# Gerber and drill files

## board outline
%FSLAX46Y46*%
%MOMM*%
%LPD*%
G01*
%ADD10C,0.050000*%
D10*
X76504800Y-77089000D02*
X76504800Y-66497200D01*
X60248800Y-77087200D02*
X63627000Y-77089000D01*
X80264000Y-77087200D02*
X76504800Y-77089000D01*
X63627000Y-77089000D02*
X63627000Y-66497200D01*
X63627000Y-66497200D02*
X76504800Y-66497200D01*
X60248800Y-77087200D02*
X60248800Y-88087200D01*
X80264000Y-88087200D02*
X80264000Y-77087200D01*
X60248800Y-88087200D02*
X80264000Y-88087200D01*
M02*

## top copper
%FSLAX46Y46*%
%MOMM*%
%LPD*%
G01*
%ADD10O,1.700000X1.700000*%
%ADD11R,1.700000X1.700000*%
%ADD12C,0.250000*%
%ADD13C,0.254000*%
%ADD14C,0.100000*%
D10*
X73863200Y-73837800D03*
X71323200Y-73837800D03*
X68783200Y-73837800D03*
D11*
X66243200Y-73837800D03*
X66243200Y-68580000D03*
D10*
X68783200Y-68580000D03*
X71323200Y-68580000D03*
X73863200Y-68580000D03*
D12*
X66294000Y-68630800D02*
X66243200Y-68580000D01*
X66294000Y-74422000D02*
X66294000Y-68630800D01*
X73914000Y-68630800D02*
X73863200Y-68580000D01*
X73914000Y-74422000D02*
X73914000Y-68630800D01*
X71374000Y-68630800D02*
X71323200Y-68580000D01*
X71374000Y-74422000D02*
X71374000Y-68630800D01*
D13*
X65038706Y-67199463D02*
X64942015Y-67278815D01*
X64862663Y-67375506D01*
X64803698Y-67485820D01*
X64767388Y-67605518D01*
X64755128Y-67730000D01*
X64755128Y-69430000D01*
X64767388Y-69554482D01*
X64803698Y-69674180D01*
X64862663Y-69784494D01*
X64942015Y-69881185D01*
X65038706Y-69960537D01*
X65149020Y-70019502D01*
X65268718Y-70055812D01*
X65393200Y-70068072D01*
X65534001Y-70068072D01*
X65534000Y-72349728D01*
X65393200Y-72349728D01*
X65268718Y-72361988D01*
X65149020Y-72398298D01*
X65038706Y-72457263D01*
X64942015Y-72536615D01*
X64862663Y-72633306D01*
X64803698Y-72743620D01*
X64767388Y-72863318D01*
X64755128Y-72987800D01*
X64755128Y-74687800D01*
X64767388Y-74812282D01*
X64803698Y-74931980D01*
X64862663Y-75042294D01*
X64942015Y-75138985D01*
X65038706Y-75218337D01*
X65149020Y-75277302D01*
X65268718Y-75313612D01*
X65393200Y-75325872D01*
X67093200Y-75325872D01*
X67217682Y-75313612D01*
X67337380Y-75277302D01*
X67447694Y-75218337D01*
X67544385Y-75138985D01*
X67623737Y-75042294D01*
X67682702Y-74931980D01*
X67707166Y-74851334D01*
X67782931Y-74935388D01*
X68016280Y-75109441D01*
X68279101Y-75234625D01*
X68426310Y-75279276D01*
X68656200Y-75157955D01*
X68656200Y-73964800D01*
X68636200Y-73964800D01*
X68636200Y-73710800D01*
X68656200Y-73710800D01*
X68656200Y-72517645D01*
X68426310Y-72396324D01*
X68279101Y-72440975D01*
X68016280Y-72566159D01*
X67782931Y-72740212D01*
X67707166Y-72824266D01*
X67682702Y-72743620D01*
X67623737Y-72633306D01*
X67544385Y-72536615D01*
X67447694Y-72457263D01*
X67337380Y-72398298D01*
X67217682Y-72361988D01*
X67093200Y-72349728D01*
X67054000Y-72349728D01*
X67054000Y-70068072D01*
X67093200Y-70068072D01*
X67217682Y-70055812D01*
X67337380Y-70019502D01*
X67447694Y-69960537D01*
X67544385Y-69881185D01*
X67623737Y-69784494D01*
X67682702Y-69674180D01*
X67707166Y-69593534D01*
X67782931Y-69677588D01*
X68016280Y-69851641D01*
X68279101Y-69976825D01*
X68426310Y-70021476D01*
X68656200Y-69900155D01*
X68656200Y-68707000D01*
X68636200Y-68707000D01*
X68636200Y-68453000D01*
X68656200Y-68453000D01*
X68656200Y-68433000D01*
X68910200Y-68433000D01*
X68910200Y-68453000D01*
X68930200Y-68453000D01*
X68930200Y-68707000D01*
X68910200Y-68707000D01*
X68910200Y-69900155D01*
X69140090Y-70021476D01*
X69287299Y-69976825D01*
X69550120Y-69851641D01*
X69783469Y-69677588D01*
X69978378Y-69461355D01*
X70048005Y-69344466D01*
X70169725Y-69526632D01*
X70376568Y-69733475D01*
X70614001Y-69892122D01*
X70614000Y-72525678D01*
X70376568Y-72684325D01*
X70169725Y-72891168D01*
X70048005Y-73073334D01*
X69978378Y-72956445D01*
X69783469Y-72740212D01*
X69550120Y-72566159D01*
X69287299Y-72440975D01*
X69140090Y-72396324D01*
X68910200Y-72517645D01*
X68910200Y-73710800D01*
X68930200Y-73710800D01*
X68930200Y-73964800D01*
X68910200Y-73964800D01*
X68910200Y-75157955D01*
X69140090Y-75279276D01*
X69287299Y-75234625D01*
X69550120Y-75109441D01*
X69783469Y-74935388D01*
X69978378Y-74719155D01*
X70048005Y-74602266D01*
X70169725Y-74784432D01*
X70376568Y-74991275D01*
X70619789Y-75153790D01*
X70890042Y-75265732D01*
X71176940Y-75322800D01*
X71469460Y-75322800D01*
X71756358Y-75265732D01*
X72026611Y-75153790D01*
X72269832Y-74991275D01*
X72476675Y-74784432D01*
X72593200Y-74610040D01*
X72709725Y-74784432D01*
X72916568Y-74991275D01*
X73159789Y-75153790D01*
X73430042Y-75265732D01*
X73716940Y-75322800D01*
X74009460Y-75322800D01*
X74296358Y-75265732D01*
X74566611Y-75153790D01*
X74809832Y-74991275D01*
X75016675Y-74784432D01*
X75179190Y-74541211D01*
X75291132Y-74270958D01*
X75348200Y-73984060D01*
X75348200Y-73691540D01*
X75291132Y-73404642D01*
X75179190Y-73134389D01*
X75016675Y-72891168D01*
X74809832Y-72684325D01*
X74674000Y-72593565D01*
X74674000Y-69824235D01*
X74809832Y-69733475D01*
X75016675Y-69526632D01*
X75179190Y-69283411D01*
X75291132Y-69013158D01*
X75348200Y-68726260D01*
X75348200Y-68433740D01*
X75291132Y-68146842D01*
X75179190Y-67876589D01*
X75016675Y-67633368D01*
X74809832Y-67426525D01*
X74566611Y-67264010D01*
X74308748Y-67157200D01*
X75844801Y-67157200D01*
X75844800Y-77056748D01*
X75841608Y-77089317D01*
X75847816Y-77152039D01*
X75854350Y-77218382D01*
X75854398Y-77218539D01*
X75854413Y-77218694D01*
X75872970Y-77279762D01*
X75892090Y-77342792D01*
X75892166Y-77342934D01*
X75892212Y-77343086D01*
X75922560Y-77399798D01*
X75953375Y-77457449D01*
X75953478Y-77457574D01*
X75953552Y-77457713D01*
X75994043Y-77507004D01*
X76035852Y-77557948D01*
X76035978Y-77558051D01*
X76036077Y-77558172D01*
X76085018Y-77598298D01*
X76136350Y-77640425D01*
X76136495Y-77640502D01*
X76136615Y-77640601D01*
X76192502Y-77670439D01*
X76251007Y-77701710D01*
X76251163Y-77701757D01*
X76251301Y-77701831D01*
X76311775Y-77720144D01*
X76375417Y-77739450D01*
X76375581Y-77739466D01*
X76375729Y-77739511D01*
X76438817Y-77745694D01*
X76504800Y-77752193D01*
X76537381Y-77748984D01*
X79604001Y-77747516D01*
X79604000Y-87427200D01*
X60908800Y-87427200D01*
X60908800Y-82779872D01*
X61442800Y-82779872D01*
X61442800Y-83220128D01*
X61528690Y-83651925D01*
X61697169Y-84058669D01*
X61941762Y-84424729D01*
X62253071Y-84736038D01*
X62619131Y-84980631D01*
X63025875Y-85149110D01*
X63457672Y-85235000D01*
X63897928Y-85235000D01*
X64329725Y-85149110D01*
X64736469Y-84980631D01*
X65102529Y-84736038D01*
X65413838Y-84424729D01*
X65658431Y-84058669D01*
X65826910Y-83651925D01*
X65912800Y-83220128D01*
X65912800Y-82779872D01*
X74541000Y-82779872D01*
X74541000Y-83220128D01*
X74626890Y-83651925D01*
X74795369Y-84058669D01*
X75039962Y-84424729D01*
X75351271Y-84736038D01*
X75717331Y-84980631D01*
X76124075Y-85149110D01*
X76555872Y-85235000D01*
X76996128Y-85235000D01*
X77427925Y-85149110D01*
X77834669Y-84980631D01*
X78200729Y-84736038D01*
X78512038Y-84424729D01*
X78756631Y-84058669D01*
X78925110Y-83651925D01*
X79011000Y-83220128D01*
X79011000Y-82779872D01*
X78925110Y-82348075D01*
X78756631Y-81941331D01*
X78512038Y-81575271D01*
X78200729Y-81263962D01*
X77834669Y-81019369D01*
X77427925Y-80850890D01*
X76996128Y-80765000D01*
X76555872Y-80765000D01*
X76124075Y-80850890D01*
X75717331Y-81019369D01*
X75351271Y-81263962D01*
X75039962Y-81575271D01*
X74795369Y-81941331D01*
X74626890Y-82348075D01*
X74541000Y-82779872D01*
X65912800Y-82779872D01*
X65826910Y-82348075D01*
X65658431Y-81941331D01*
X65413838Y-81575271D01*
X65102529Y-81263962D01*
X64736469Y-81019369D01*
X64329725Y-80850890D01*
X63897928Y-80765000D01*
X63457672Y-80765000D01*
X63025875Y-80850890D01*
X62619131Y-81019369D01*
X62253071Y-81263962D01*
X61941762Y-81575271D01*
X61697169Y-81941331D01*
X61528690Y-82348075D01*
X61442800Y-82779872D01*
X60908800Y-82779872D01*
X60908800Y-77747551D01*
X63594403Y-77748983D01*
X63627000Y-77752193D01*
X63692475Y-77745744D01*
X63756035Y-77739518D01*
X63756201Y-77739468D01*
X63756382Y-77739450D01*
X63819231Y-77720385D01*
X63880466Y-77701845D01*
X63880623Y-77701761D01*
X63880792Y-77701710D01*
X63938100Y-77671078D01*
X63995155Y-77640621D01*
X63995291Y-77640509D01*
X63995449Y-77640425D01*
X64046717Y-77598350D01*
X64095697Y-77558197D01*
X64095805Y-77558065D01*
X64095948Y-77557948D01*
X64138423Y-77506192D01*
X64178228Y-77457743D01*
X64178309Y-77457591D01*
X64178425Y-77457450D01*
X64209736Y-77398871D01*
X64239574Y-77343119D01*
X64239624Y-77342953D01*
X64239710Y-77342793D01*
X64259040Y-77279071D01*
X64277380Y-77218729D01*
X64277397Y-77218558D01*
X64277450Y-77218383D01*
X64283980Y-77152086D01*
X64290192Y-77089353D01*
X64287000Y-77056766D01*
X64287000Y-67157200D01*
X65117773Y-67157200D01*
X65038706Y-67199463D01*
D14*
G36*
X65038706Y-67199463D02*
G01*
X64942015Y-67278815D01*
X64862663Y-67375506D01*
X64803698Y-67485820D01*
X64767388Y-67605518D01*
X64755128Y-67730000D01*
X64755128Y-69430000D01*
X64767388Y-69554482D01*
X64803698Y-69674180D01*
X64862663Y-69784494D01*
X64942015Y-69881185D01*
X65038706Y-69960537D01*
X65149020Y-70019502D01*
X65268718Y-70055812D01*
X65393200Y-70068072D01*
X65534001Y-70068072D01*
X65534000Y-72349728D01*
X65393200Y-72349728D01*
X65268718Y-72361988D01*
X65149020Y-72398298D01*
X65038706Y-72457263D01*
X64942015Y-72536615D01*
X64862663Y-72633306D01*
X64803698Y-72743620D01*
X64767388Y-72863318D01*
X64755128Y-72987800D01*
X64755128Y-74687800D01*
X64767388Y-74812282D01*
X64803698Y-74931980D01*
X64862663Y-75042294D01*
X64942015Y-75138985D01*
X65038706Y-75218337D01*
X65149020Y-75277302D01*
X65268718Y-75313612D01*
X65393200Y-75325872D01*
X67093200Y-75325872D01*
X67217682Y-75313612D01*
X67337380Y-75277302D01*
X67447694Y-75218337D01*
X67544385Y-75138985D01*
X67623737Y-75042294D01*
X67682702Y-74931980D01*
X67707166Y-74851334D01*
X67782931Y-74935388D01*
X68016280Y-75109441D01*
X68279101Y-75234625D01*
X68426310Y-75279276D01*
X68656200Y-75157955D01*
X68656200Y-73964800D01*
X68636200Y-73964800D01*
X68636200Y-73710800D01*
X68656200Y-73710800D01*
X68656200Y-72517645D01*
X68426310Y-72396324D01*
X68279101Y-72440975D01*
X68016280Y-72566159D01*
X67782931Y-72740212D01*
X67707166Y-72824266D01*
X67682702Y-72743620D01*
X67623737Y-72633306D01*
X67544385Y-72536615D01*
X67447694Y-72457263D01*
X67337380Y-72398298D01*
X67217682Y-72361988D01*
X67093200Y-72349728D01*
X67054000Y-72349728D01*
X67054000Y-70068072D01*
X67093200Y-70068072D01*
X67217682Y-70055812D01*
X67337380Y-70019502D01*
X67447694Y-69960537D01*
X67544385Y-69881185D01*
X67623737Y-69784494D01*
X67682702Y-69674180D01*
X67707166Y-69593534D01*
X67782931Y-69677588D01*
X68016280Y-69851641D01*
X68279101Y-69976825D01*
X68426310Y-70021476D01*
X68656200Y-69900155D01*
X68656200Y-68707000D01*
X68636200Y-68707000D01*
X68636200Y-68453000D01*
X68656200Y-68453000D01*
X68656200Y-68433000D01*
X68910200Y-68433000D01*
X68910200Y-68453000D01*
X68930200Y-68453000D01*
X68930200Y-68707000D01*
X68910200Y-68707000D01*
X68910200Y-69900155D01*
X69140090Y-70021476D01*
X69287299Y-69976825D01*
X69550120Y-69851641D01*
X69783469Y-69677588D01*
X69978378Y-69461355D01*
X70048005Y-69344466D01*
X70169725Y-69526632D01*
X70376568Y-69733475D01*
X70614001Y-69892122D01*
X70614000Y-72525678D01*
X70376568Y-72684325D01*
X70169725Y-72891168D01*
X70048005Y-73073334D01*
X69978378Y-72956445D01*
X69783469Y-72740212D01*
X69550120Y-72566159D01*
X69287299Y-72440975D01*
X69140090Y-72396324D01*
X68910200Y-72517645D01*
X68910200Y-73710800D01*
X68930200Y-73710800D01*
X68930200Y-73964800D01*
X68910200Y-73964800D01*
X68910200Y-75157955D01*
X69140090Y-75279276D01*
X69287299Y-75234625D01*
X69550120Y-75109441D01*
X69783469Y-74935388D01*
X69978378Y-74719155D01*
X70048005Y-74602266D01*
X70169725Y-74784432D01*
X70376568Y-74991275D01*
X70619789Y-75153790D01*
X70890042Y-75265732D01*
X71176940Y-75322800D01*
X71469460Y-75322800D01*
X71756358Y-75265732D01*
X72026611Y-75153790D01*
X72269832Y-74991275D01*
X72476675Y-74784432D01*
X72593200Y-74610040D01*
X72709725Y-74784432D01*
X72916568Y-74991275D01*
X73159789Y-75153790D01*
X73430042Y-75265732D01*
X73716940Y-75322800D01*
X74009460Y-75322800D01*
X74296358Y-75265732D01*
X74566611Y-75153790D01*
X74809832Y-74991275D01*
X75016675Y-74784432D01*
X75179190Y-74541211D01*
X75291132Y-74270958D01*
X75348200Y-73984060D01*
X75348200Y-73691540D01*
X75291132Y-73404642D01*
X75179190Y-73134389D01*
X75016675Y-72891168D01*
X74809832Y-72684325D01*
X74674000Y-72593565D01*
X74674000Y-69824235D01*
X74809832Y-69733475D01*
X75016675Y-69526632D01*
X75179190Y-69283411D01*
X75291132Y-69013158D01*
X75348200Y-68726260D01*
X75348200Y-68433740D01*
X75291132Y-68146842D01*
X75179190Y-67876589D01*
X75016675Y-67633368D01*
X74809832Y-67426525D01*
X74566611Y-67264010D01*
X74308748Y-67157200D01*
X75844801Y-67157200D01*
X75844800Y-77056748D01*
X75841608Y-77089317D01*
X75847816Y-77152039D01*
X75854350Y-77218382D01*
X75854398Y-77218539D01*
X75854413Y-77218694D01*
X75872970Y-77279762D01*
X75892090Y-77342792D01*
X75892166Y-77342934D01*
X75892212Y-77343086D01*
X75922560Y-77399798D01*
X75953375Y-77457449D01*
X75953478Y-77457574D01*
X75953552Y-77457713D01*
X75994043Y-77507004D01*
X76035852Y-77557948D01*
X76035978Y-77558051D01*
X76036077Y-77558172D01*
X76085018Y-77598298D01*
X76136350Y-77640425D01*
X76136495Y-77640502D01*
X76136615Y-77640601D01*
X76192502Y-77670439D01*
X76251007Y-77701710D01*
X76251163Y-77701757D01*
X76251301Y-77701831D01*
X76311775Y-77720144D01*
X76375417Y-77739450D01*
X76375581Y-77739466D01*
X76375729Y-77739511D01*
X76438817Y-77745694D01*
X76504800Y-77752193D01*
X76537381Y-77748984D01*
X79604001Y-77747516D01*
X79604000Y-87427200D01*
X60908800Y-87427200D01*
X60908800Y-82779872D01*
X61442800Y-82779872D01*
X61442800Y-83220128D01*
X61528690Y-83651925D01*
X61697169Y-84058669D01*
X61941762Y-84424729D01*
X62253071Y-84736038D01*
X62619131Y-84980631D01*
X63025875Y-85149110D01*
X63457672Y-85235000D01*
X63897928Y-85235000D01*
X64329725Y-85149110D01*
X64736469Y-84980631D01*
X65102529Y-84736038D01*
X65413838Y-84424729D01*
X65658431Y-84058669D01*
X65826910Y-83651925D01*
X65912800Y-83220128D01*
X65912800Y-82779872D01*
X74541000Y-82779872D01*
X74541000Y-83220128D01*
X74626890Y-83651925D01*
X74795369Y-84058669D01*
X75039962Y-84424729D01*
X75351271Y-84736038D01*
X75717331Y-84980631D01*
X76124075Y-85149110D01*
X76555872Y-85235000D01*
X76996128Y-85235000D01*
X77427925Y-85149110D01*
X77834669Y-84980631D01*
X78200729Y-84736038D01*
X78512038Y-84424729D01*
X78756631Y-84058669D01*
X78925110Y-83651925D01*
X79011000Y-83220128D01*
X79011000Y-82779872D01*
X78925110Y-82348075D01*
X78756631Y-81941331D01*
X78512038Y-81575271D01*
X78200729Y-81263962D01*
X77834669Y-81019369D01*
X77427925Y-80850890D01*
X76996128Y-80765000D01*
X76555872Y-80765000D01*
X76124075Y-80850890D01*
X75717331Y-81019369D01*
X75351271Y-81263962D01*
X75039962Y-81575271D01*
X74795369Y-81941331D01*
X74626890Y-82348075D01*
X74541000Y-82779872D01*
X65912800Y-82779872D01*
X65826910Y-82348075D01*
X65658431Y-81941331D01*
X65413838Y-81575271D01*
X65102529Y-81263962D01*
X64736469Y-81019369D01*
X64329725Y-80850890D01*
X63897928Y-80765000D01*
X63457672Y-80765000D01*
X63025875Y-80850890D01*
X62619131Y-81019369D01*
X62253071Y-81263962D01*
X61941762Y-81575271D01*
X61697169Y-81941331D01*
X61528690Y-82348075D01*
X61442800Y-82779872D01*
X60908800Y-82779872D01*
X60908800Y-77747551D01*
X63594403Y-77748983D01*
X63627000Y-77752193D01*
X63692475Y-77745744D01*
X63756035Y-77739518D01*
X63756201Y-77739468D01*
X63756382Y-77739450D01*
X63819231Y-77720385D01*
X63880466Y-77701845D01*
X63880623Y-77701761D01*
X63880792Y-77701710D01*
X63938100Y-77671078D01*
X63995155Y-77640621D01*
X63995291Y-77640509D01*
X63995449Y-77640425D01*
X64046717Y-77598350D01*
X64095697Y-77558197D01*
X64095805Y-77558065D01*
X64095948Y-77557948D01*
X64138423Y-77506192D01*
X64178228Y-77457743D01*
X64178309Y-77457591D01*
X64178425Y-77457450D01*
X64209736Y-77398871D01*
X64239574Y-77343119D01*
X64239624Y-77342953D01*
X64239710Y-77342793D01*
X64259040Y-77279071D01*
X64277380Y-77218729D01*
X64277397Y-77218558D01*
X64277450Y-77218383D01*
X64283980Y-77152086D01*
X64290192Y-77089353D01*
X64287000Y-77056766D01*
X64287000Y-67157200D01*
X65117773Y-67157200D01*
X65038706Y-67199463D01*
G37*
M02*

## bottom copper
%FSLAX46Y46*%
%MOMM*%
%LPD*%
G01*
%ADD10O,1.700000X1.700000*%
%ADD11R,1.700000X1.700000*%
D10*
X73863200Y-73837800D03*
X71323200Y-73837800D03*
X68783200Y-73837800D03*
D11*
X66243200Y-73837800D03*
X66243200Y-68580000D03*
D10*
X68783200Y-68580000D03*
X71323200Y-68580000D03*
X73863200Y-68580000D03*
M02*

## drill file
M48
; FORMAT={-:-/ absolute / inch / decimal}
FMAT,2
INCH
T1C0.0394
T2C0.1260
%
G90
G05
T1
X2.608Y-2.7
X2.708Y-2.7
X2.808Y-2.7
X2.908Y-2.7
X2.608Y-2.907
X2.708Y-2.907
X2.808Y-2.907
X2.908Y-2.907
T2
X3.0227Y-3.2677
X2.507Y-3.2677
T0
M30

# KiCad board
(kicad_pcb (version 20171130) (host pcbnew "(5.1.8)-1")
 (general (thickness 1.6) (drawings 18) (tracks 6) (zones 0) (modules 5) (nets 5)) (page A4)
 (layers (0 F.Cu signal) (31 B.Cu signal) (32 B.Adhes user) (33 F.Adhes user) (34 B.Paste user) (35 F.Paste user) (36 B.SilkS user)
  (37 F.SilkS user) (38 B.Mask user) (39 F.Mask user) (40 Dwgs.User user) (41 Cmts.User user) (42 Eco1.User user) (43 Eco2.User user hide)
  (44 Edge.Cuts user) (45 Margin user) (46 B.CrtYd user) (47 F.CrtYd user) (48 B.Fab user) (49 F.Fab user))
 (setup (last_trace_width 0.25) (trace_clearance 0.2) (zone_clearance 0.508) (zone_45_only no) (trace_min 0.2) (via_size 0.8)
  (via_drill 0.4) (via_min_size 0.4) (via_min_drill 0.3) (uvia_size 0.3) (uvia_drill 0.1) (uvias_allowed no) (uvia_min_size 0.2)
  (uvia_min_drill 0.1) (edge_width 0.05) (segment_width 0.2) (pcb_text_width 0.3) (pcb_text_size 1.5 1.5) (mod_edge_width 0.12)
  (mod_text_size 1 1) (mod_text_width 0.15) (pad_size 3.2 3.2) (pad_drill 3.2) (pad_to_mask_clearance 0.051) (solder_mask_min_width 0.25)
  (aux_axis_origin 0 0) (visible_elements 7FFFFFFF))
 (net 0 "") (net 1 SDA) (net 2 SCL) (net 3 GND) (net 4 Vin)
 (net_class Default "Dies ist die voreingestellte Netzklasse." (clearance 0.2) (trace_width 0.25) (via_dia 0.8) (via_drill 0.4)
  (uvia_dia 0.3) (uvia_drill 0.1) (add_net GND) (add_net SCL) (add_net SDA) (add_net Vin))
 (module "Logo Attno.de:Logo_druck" (layer F.Cu) (at 70.0786 81.6356)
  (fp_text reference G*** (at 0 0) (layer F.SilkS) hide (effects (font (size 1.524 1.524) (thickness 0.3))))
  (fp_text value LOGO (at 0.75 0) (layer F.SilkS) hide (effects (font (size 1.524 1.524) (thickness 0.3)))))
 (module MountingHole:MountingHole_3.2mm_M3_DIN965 (layer F.Cu) (at 76.776 83)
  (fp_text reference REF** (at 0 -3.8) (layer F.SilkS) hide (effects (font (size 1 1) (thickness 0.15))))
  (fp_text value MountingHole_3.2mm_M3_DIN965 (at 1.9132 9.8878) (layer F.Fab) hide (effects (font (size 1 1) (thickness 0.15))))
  (pad 1 np_thru_hole circle (at 0 0) (size 3.2 3.2) (drill 3.2) (layers *.Cu *.Mask)))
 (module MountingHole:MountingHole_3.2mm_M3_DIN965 (layer F.Cu) (at 63.6778 83)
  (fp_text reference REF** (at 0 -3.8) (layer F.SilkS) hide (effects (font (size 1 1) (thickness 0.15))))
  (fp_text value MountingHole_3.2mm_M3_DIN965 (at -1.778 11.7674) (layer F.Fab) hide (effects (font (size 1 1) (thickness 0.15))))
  (pad 1 np_thru_hole circle (at 0 0) (size 3.2 3.2) (drill 3.2) (layers *.Cu *.Mask)))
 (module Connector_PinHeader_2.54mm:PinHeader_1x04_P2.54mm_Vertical (layer F.Cu) (at 66.2432 73.8378 90)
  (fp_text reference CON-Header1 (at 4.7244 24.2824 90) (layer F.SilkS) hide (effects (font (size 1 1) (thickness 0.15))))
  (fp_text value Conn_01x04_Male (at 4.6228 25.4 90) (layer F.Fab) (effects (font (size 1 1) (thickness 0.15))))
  (pad 4 thru_hole oval (at 0 7.62 90) (size 1.7 1.7) (drill 1) (layers *.Cu *.Mask) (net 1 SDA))
  (pad 3 thru_hole oval (at 0 5.08 90) (size 1.7 1.7) (drill 1) (layers *.Cu *.Mask) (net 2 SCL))
  (pad 2 thru_hole oval (at 0 2.54 90) (size 1.7 1.7) (drill 1) (layers *.Cu *.Mask) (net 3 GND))
  (pad 1 thru_hole rect (at 0 0 90) (size 1.7 1.7) (drill 1) (layers *.Cu *.Mask) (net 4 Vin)))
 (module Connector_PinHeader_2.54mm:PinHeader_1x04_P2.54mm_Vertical (layer F.Cu) (at 66.2432 68.58 90)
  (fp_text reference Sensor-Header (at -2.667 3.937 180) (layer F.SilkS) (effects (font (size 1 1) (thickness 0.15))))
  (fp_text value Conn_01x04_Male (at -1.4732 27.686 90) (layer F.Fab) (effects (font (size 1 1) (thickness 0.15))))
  (pad 1 thru_hole rect (at 0 0 90) (size 1.7 1.7) (drill 1) (layers *.Cu *.Mask) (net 4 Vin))
  (pad 2 thru_hole oval (at 0 2.54 90) (size 1.7 1.7) (drill 1) (layers *.Cu *.Mask) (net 3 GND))
  (pad 3 thru_hole oval (at 0 5.08 90) (size 1.7 1.7) (drill 1) (layers *.Cu *.Mask) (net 2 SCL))
  (pad 4 thru_hole oval (at 0 7.62 90) (size 1.7 1.7) (drill 1) (layers *.Cu *.Mask) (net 1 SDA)))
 (gr_line (start 76.5048 77.089) (end 76.5048 66.4972) (layer Edge.Cuts) (width 0.05))
 (gr_line (start 60.2488 77.0872) (end 63.627 77.089) (layer Edge.Cuts) (width 0.05))
 (gr_line (start 80.264 77.0872) (end 76.5048 77.089) (layer Edge.Cuts) (width 0.05))
 (gr_line (start 63.627 77.089) (end 63.627 66.4972) (layer Edge.Cuts) (width 0.05))
 (gr_line (start 63.627 66.4972) (end 76.5048 66.4972) (layer Edge.Cuts) (width 0.05))
 (gr_line (start 60.2488 77.0872) (end 60.2488 88.0872) (layer Edge.Cuts) (width 0.05))
 (gr_line (start 80.264 88.0872) (end 80.264 77.0872) (layer Edge.Cuts) (width 0.05))
 (gr_line (start 60.2488 88.0872) (end 80.264 88.0872) (layer Edge.Cuts) (width 0.05))
 (segment (start 66.294 68.6308) (end 66.2432 68.58) (width 0.25) (layer F.Cu) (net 4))
 (segment (start 66.294 74.422) (end 66.294 68.6308) (width 0.25) (layer F.Cu) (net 4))
 (segment (start 73.914 68.6308) (end 73.8632 68.58) (width 0.25) (layer F.Cu) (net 1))
 (segment (start 73.914 74.422) (end 73.914 68.6308) (width 0.25) (layer F.Cu) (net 1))
 (segment (start 71.374 68.6308) (end 71.3232 68.58) (width 0.25) (layer F.Cu) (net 2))
 (segment (start 71.374 74.422) (end 71.374 68.6308) (width 0.25) (layer F.Cu) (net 2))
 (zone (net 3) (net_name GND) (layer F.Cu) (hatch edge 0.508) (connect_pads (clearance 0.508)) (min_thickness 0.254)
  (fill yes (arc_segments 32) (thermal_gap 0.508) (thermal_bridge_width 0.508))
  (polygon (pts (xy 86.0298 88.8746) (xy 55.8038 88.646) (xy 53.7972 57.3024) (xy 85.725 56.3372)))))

